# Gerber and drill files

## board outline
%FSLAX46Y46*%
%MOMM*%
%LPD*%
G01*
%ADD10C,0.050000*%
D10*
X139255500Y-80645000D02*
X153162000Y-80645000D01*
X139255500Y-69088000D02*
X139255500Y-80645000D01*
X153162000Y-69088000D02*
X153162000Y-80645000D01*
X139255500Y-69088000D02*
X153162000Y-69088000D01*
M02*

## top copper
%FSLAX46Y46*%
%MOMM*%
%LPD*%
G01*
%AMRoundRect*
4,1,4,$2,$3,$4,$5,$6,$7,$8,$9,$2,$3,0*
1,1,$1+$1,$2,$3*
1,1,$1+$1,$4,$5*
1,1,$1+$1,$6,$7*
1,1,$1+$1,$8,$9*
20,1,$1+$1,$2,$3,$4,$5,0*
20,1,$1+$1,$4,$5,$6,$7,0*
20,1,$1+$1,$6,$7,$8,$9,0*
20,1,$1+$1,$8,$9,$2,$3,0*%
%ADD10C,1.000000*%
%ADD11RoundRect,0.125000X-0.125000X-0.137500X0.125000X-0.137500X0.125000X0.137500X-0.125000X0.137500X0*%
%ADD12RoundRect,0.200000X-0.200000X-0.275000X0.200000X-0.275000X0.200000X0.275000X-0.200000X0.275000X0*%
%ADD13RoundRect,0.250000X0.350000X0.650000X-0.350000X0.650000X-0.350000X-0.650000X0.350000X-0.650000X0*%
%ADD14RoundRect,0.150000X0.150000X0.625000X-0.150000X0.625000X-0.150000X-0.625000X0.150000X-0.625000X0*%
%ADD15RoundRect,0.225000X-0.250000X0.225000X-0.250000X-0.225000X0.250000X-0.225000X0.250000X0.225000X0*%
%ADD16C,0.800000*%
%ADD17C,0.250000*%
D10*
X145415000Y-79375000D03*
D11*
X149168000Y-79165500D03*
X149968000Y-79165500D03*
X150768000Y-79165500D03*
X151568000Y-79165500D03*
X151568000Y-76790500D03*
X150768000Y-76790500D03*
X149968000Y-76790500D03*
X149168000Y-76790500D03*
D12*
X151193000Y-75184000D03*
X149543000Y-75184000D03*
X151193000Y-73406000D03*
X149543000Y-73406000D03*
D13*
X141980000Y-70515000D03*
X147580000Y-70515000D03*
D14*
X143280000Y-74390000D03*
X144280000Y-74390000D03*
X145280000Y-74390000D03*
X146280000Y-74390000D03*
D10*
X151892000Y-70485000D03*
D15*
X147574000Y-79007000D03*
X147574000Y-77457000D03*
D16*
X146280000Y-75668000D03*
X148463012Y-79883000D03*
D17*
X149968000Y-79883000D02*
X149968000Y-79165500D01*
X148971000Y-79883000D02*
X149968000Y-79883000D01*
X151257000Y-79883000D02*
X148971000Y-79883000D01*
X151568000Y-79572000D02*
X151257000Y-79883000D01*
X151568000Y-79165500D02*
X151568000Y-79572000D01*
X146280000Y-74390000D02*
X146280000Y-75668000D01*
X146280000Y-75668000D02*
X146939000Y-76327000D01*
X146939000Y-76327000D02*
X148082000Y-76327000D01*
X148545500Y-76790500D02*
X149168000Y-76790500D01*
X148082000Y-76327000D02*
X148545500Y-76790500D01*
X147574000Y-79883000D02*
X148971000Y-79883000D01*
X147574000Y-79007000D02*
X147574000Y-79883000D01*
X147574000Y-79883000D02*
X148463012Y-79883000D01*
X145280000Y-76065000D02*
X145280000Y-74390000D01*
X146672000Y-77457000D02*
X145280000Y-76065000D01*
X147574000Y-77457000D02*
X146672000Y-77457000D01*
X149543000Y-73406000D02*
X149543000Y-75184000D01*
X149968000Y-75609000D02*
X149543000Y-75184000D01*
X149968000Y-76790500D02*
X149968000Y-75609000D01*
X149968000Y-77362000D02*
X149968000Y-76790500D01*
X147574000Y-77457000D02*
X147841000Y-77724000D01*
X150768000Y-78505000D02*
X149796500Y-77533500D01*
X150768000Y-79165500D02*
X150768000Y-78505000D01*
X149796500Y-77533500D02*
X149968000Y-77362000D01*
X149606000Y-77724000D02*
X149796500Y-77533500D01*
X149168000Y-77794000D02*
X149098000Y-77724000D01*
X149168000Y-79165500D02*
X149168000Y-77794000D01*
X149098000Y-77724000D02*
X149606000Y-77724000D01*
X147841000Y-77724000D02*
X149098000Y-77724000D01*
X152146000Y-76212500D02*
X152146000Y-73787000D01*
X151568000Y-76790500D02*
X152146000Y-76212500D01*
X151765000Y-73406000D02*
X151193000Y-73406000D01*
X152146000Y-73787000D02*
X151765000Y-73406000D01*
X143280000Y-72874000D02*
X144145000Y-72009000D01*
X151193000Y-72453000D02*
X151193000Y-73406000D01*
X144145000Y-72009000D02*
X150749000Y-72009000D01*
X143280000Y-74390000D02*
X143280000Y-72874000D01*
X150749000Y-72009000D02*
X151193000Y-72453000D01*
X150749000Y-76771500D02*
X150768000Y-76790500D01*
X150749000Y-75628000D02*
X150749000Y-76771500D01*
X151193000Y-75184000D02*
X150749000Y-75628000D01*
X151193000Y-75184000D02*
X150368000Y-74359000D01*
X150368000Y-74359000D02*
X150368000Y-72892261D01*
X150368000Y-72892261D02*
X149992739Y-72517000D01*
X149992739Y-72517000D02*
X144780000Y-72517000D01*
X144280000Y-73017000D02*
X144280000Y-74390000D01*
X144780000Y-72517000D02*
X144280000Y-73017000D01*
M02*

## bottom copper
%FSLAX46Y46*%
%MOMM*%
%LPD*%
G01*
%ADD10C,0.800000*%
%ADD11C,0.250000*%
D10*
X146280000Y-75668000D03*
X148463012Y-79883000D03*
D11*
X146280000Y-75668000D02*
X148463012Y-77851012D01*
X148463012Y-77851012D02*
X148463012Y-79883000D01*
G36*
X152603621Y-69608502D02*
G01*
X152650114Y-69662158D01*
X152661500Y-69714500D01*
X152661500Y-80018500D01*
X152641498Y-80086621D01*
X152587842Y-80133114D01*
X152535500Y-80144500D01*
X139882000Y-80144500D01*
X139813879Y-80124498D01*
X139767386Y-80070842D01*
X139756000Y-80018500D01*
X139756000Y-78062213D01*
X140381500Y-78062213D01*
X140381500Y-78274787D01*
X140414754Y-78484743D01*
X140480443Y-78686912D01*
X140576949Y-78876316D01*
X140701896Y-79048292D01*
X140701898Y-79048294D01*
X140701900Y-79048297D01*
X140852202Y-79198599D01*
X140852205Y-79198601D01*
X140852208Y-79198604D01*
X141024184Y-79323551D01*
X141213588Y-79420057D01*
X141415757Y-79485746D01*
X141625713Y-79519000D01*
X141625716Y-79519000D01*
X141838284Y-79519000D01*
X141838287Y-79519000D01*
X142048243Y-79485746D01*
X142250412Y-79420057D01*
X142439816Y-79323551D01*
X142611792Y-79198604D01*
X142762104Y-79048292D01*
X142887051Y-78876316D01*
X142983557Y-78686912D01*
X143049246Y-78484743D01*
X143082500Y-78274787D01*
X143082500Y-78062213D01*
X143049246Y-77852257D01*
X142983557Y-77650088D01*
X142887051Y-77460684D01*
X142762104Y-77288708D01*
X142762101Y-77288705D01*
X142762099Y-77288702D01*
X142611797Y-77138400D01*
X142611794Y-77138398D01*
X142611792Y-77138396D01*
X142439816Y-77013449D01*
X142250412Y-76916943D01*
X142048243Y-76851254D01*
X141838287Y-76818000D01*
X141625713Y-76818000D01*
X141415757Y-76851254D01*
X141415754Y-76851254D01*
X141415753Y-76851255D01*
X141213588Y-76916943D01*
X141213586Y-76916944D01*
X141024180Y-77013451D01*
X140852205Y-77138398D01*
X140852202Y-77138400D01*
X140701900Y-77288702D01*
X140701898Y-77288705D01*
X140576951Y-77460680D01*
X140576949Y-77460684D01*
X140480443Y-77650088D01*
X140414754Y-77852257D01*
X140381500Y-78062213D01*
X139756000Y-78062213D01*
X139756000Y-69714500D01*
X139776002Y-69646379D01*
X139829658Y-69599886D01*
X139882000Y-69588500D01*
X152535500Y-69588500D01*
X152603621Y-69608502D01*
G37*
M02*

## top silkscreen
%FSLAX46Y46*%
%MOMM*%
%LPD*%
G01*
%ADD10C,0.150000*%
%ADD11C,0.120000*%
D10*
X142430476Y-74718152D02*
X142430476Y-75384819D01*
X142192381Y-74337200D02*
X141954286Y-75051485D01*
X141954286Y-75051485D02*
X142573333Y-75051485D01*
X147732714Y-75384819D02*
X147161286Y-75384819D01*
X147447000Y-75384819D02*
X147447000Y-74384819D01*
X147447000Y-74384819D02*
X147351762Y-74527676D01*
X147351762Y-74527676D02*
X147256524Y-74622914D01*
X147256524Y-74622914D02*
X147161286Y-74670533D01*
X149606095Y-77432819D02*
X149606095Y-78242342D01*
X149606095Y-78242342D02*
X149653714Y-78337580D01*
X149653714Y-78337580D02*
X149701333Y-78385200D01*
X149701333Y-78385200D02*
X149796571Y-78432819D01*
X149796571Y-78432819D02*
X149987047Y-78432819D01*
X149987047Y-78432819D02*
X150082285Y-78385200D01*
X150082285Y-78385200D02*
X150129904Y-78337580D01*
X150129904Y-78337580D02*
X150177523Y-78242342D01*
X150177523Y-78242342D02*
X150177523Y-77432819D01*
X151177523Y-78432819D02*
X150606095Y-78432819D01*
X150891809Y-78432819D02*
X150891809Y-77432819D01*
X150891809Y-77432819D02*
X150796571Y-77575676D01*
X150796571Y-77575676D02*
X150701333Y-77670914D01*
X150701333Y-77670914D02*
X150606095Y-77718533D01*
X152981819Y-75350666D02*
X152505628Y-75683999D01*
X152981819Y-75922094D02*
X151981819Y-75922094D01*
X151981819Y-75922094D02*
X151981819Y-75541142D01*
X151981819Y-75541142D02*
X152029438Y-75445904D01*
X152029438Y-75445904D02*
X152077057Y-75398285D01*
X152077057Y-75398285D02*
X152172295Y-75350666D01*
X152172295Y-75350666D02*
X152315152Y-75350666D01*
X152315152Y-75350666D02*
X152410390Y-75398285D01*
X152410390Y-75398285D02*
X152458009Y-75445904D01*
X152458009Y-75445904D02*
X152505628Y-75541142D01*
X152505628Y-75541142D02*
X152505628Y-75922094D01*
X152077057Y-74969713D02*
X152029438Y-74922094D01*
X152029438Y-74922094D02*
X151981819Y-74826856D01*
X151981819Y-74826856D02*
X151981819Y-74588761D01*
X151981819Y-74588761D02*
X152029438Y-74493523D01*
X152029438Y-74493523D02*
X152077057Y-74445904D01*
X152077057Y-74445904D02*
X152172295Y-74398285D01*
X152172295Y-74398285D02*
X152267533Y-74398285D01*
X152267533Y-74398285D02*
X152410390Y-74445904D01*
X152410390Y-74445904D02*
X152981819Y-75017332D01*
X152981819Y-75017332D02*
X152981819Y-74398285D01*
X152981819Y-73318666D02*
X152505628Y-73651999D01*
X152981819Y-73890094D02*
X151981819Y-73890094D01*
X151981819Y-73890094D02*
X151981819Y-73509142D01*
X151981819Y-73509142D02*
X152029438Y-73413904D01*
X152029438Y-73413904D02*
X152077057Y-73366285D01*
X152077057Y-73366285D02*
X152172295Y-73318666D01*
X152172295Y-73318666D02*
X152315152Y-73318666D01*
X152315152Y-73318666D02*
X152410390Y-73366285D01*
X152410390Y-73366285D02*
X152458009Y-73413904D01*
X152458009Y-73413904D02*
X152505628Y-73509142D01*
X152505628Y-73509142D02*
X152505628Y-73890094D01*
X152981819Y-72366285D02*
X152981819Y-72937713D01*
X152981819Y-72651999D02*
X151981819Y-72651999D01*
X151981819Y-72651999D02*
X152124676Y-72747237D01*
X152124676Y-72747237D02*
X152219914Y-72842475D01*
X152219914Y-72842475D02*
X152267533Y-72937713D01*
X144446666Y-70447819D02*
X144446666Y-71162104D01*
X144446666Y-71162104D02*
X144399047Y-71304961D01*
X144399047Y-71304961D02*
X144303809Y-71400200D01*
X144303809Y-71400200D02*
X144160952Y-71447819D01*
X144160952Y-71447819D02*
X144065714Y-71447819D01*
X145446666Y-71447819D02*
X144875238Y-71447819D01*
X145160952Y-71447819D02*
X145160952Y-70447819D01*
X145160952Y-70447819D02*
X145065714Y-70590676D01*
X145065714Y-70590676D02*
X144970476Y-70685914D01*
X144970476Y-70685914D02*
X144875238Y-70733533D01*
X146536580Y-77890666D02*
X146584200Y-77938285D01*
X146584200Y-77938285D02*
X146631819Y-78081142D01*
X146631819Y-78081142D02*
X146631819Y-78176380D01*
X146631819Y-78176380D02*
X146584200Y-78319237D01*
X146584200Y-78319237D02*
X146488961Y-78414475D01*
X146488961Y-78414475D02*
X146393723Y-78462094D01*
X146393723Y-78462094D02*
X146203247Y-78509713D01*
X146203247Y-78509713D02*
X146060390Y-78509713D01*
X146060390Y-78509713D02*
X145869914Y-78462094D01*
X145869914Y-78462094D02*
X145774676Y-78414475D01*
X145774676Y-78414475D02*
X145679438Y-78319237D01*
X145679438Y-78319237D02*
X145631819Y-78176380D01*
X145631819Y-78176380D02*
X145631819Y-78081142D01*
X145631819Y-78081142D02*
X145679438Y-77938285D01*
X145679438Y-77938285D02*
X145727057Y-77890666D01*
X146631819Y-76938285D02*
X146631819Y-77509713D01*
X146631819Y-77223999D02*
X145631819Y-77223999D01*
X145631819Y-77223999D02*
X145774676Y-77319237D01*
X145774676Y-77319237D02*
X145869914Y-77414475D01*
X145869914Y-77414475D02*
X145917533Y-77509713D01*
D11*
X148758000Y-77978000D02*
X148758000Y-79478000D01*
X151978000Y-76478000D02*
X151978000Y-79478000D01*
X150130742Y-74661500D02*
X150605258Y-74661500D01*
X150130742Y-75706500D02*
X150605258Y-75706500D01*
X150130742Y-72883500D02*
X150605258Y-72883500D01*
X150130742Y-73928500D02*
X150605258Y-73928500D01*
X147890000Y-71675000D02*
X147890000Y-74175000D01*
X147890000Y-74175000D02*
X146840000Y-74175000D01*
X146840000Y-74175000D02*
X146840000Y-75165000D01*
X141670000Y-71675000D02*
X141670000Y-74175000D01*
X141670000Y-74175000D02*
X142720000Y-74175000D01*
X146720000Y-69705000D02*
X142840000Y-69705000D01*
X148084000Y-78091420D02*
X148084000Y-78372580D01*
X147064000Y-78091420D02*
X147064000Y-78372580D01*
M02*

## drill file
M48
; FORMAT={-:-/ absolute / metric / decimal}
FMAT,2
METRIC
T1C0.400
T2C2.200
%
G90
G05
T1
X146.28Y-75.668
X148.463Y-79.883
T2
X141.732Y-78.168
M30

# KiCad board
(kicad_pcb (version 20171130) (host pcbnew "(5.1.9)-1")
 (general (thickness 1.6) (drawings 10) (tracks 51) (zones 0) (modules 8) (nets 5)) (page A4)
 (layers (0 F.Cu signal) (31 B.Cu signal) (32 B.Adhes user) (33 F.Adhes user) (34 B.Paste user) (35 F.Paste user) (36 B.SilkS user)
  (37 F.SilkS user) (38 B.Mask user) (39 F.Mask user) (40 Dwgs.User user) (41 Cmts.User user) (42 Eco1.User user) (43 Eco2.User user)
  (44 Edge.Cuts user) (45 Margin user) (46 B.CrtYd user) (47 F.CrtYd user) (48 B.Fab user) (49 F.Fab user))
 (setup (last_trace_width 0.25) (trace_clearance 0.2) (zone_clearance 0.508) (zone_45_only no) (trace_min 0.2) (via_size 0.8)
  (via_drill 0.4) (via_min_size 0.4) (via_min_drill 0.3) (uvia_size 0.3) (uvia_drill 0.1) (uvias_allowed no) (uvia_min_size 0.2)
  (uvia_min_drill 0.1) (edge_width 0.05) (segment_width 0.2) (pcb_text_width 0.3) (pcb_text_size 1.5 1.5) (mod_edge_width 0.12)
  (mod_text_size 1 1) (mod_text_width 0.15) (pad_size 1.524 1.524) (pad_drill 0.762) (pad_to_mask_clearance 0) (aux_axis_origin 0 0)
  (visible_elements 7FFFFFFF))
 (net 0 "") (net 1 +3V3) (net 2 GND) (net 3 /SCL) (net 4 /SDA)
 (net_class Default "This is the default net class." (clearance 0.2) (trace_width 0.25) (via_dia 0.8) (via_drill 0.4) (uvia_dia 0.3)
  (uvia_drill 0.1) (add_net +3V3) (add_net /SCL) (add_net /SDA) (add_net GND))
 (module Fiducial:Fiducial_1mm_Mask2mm (layer F.Cu) (at 145.415 79.375)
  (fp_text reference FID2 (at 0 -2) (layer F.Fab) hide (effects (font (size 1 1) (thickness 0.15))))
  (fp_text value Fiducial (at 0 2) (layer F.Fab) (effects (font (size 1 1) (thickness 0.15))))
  (pad "" smd circle (at 0 0) (size 1 1) (layers F.Cu F.Mask) (solder_mask_margin 0.5) (clearance 0.5)))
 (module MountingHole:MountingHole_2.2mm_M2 (layer F.Cu) (at 141.732 78.1685)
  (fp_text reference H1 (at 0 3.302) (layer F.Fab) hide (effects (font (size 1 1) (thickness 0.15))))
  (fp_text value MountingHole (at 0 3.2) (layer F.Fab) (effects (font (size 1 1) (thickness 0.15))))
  (pad 1 np_thru_hole circle (at 0 0) (size 2.2 2.2) (drill 2.2) (layers *.Cu *.Mask)))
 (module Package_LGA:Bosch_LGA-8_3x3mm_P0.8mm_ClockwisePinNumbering (layer F.Cu) (at 150.368 77.978)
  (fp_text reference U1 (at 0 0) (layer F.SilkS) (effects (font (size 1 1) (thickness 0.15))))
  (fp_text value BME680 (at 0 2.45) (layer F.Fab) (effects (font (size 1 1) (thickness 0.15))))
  (fp_line (start -1.61 0) (end -1.61 1.5) (layer F.SilkS) (width 0.12))
  (fp_line (start 1.61 -1.5) (end 1.61 1.5) (layer F.SilkS) (width 0.12))
  (pad 8 smd roundrect (at -1.2 1.1875) (size 0.5 0.525) (layers F.Cu F.Paste F.Mask) (roundrect_rratio 0.25) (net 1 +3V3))
  (pad 7 smd roundrect (at -0.4 1.1875) (size 0.5 0.525) (layers F.Cu F.Paste F.Mask) (roundrect_rratio 0.25) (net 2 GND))
  (pad 6 smd roundrect (at 0.4 1.1875) (size 0.5 0.525) (layers F.Cu F.Paste F.Mask) (roundrect_rratio 0.25) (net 1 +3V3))
  (pad 5 smd roundrect (at 1.2 1.1875) (size 0.5 0.525) (layers F.Cu F.Paste F.Mask) (roundrect_rratio 0.25) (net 2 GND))
  (pad 4 smd roundrect (at 1.2 -1.1875) (size 0.5 0.525) (layers F.Cu F.Paste F.Mask) (roundrect_rratio 0.25) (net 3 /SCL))
  (pad 3 smd roundrect (at 0.4 -1.1875) (size 0.5 0.525) (layers F.Cu F.Paste F.Mask) (roundrect_rratio 0.25) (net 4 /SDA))
  (pad 2 smd roundrect (at -0.4 -1.1875) (size 0.5 0.525) (layers F.Cu F.Paste F.Mask) (roundrect_rratio 0.25) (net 1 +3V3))
  (pad 1 smd roundrect (at -1.2 -1.1875) (size 0.5 0.525) (layers F.Cu F.Paste F.Mask) (roundrect_rratio 0.25) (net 2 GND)))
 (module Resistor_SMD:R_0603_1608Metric (layer F.Cu) (at 150.368 75.184)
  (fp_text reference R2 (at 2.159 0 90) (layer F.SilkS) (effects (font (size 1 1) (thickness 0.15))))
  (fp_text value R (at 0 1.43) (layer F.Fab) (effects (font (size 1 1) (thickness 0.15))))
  (fp_line (start -0.237258 -0.5225) (end 0.237258 -0.5225) (layer F.SilkS) (width 0.12))
  (fp_line (start -0.237258 0.5225) (end 0.237258 0.5225) (layer F.SilkS) (width 0.12))
  (pad 2 smd roundrect (at 0.825 0) (size 0.8 0.95) (layers F.Cu F.Paste F.Mask) (roundrect_rratio 0.25) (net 4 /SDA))
  (pad 1 smd roundrect (at -0.825 0) (size 0.8 0.95) (layers F.Cu F.Paste F.Mask) (roundrect_rratio 0.25) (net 1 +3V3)))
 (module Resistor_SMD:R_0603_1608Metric (layer F.Cu) (at 150.368 73.406)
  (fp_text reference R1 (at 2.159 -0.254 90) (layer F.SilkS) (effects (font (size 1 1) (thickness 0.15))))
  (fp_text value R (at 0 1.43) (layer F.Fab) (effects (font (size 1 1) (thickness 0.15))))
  (fp_line (start -0.237258 -0.5225) (end 0.237258 -0.5225) (layer F.SilkS) (width 0.12))
  (fp_line (start -0.237258 0.5225) (end 0.237258 0.5225) (layer F.SilkS) (width 0.12))
  (pad 2 smd roundrect (at 0.825 0) (size 0.8 0.95) (layers F.Cu F.Paste F.Mask) (roundrect_rratio 0.25) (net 3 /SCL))
  (pad 1 smd roundrect (at -0.825 0) (size 0.8 0.95) (layers F.Cu F.Paste F.Mask) (roundrect_rratio 0.25) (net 1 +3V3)))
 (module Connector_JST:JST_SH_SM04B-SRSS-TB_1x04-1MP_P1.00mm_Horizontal (layer F.Cu) (at 144.78 72.39 180)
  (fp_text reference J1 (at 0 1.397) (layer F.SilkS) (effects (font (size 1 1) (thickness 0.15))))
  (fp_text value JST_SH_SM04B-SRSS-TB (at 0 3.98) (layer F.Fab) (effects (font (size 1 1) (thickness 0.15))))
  (fp_line (start -3.11 0.715) (end -3.11 -1.785) (layer F.SilkS) (width 0.12))
  (fp_line (start -3.11 -1.785) (end -2.06 -1.785) (layer F.SilkS) (width 0.12))
  (fp_line (start -2.06 -1.785) (end -2.06 -2.775) (layer F.SilkS) (width 0.12))
  (fp_line (start 3.11 0.715) (end 3.11 -1.785) (layer F.SilkS) (width 0.12))
  (fp_line (start 3.11 -1.785) (end 2.06 -1.785) (layer F.SilkS) (width 0.12))
  (fp_line (start -1.94 2.685) (end 1.94 2.685) (layer F.SilkS) (width 0.12))
  (pad MP smd roundrect (at 2.8 1.875 180) (size 1.2 1.8) (layers F.Cu F.Paste F.Mask) (roundrect_rratio 0.208333))
  (pad MP smd roundrect (at -2.8 1.875 180) (size 1.2 1.8) (layers F.Cu F.Paste F.Mask) (roundrect_rratio 0.208333))
  (pad 4 smd roundrect (at 1.5 -2 180) (size 0.6 1.55) (layers F.Cu F.Paste F.Mask) (roundrect_rratio 0.25) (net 3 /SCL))
  (pad 3 smd roundrect (at 0.5 -2 180) (size 0.6 1.55) (layers F.Cu F.Paste F.Mask) (roundrect_rratio 0.25) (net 4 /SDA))
  (pad 2 smd roundrect (at -0.5 -2 180) (size 0.6 1.55) (layers F.Cu F.Paste F.Mask) (roundrect_rratio 0.25) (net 1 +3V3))
  (pad 1 smd roundrect (at -1.5 -2 180) (size 0.6 1.55) (layers F.Cu F.Paste F.Mask) (roundrect_rratio 0.25) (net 2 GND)))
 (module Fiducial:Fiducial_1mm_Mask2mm (layer F.Cu) (at 151.892 70.485)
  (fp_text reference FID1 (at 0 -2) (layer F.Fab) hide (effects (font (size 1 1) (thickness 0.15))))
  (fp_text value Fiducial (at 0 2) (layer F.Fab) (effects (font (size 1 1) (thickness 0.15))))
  (pad "" smd circle (at 0 0) (size 1 1) (layers F.Cu F.Mask) (solder_mask_margin 0.5) (clearance 0.5)))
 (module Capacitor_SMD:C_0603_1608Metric (layer F.Cu) (at 147.574 78.232 270)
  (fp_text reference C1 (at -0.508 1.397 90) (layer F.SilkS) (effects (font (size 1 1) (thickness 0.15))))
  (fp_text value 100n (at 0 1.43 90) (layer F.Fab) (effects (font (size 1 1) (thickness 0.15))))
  (fp_line (start -0.14058 -0.51) (end 0.14058 -0.51) (layer F.SilkS) (width 0.12))
  (fp_line (start -0.14058 0.51) (end 0.14058 0.51) (layer F.SilkS) (width 0.12))
  (pad 2 smd roundrect (at 0.775 0 270) (size 0.9 0.95) (layers F.Cu F.Paste F.Mask) (roundrect_rratio 0.25) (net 2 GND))
  (pad 1 smd roundrect (at -0.775 0 270) (size 0.9 0.95) (layers F.Cu F.Paste F.Mask) (roundrect_rratio 0.25) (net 1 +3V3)))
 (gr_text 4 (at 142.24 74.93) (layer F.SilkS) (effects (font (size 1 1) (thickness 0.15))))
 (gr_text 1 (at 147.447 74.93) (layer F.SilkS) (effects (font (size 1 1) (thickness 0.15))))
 (gr_line (start 139.2555 80.645) (end 153.162 80.645) (layer Edge.Cuts) (width 0.05))
 (gr_line (start 139.2555 69.088) (end 139.2555 80.645) (layer Edge.Cuts) (width 0.05))
 (gr_line (start 153.162 69.088) (end 153.162 80.645) (layer Edge.Cuts) (width 0.05))
 (gr_line (start 139.2555 69.088) (end 153.162 69.088) (layer Edge.Cuts) (width 0.05))
 (segment (start 149.968 79.883) (end 149.968 79.1655) (width 0.25) (layer F.Cu) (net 2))
 (segment (start 148.971 79.883) (end 149.968 79.883) (width 0.25) (layer F.Cu) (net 2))
 (segment (start 151.257 79.883) (end 148.971 79.883) (width 0.25) (layer F.Cu) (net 2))
 (segment (start 151.568 79.572) (end 151.257 79.883) (width 0.25) (layer F.Cu) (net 2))
 (segment (start 151.568 79.1655) (end 151.568 79.572) (width 0.25) (layer F.Cu) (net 2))
 (segment (start 146.28 74.39) (end 146.28 75.668) (width 0.25) (layer F.Cu) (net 2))
 (segment (start 146.28 75.668) (end 146.939 76.327) (width 0.25) (layer F.Cu) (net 2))
 (segment (start 146.939 76.327) (end 148.082 76.327) (width 0.25) (layer F.Cu) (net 2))
 (segment (start 148.5455 76.7905) (end 149.168 76.7905) (width 0.25) (layer F.Cu) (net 2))
 (segment (start 148.082 76.327) (end 148.5455 76.7905) (width 0.25) (layer F.Cu) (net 2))
 (via (at 146.28 75.668) (size 0.8) (drill 0.4) (layers F.Cu B.Cu) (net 2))
 (segment (start 147.574 79.883) (end 148.971 79.883) (width 0.25) (layer F.Cu) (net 2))
 (segment (start 147.574 79.007) (end 147.574 79.883) (width 0.25) (layer F.Cu) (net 2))
 (segment (start 147.574 79.883) (end 148.463012 79.883) (width 0.25) (layer F.Cu) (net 2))
 (via (at 148.463012 79.883) (size 0.8) (drill 0.4) (layers F.Cu B.Cu) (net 2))
 (segment (start 146.28 75.668) (end 148.463012 77.851012) (width 0.25) (layer B.Cu) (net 2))
 (segment (start 148.463012 77.851012) (end 148.463012 79.883) (width 0.25) (layer B.Cu) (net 2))
 (segment (start 145.28 76.065) (end 145.28 74.39) (width 0.25) (layer F.Cu) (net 1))
 (segment (start 146.672 77.457) (end 145.28 76.065) (width 0.25) (layer F.Cu) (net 1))
 (segment (start 147.574 77.457) (end 146.672 77.457) (width 0.25) (layer F.Cu) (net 1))
 (segment (start 149.543 73.406) (end 149.543 75.184) (width 0.25) (layer F.Cu) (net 1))
 (segment (start 149.968 75.609) (end 149.543 75.184) (width 0.25) (layer F.Cu) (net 1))
 (segment (start 149.968 76.7905) (end 149.968 75.609) (width 0.25) (layer F.Cu) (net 1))
 (segment (start 149.968 77.362) (end 149.968 76.7905) (width 0.25) (layer F.Cu) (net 1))
 (segment (start 147.574 77.457) (end 147.841 77.724) (width 0.25) (layer F.Cu) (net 1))
 (segment (start 150.768 78.505) (end 149.7965 77.5335) (width 0.25) (layer F.Cu) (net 1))
 (segment (start 150.768 79.1655) (end 150.768 78.505) (width 0.25) (layer F.Cu) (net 1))
 (segment (start 149.7965 77.5335) (end 149.968 77.362) (width 0.25) (layer F.Cu) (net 1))
 (segment (start 149.606 77.724) (end 149.7965 77.5335) (width 0.25) (layer F.Cu) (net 1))
 (segment (start 149.168 77.794) (end 149.098 77.724) (width 0.25) (layer F.Cu) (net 1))
 (segment (start 149.168 79.1655) (end 149.168 77.794) (width 0.25) (layer F.Cu) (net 1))
 (segment (start 149.098 77.724) (end 149.606 77.724) (width 0.25) (layer F.Cu) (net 1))
 (segment (start 147.841 77.724) (end 149.098 77.724) (width 0.25) (layer F.Cu) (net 1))
 (segment (start 152.146 76.2125) (end 152.146 73.787) (width 0.25) (layer F.Cu) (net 3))
 (segment (start 151.568 76.7905) (end 152.146 76.2125) (width 0.25) (layer F.Cu) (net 3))
 (segment (start 151.765 73.406) (end 151.193 73.406) (width 0.25) (layer F.Cu) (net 3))
 (segment (start 152.146 73.787) (end 151.765 73.406) (width 0.25) (layer F.Cu) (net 3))
 (segment (start 143.28 72.874) (end 144.145 72.009) (width 0.25) (layer F.Cu) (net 3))
 (segment (start 151.193 72.453) (end 151.193 73.406) (width 0.25) (layer F.Cu) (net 3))
 (segment (start 144.145 72.009) (end 150.749 72.009) (width 0.25) (layer F.Cu) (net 3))
 (segment (start 143.28 74.39) (end 143.28 72.874) (width 0.25) (layer F.Cu) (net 3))
 (segment (start 150.749 72.009) (end 151.193 72.453) (width 0.25) (layer F.Cu) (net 3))
 (segment (start 150.749 76.7715) (end 150.768 76.7905) (width 0.25) (layer F.Cu) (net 4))
 (segment (start 150.749 75.628) (end 150.749 76.7715) (width 0.25) (layer F.Cu) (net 4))
 (segment (start 151.193 75.184) (end 150.749 75.628) (width 0.25) (layer F.Cu) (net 4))
 (segment (start 151.193 75.184) (end 150.368 74.359) (width 0.25) (layer F.Cu) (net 4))
 (segment (start 150.368 74.359) (end 150.368 72.892261) (width 0.25) (layer F.Cu) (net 4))
 (segment (start 150.368 72.892261) (end 149.992739 72.517) (width 0.25) (layer F.Cu) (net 4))
 (segment (start 149.992739 72.517) (end 144.78 72.517) (width 0.25) (layer F.Cu) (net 4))
 (segment (start 144.28 73.017) (end 144.28 74.39) (width 0.25) (layer F.Cu) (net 4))
 (segment (start 144.78 72.517) (end 144.28 73.017) (width 0.25) (layer F.Cu) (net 4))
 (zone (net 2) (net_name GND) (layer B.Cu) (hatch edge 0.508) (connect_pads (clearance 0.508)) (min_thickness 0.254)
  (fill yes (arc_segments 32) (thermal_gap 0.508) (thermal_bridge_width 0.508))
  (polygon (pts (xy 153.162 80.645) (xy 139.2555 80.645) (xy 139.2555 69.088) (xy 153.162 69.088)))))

